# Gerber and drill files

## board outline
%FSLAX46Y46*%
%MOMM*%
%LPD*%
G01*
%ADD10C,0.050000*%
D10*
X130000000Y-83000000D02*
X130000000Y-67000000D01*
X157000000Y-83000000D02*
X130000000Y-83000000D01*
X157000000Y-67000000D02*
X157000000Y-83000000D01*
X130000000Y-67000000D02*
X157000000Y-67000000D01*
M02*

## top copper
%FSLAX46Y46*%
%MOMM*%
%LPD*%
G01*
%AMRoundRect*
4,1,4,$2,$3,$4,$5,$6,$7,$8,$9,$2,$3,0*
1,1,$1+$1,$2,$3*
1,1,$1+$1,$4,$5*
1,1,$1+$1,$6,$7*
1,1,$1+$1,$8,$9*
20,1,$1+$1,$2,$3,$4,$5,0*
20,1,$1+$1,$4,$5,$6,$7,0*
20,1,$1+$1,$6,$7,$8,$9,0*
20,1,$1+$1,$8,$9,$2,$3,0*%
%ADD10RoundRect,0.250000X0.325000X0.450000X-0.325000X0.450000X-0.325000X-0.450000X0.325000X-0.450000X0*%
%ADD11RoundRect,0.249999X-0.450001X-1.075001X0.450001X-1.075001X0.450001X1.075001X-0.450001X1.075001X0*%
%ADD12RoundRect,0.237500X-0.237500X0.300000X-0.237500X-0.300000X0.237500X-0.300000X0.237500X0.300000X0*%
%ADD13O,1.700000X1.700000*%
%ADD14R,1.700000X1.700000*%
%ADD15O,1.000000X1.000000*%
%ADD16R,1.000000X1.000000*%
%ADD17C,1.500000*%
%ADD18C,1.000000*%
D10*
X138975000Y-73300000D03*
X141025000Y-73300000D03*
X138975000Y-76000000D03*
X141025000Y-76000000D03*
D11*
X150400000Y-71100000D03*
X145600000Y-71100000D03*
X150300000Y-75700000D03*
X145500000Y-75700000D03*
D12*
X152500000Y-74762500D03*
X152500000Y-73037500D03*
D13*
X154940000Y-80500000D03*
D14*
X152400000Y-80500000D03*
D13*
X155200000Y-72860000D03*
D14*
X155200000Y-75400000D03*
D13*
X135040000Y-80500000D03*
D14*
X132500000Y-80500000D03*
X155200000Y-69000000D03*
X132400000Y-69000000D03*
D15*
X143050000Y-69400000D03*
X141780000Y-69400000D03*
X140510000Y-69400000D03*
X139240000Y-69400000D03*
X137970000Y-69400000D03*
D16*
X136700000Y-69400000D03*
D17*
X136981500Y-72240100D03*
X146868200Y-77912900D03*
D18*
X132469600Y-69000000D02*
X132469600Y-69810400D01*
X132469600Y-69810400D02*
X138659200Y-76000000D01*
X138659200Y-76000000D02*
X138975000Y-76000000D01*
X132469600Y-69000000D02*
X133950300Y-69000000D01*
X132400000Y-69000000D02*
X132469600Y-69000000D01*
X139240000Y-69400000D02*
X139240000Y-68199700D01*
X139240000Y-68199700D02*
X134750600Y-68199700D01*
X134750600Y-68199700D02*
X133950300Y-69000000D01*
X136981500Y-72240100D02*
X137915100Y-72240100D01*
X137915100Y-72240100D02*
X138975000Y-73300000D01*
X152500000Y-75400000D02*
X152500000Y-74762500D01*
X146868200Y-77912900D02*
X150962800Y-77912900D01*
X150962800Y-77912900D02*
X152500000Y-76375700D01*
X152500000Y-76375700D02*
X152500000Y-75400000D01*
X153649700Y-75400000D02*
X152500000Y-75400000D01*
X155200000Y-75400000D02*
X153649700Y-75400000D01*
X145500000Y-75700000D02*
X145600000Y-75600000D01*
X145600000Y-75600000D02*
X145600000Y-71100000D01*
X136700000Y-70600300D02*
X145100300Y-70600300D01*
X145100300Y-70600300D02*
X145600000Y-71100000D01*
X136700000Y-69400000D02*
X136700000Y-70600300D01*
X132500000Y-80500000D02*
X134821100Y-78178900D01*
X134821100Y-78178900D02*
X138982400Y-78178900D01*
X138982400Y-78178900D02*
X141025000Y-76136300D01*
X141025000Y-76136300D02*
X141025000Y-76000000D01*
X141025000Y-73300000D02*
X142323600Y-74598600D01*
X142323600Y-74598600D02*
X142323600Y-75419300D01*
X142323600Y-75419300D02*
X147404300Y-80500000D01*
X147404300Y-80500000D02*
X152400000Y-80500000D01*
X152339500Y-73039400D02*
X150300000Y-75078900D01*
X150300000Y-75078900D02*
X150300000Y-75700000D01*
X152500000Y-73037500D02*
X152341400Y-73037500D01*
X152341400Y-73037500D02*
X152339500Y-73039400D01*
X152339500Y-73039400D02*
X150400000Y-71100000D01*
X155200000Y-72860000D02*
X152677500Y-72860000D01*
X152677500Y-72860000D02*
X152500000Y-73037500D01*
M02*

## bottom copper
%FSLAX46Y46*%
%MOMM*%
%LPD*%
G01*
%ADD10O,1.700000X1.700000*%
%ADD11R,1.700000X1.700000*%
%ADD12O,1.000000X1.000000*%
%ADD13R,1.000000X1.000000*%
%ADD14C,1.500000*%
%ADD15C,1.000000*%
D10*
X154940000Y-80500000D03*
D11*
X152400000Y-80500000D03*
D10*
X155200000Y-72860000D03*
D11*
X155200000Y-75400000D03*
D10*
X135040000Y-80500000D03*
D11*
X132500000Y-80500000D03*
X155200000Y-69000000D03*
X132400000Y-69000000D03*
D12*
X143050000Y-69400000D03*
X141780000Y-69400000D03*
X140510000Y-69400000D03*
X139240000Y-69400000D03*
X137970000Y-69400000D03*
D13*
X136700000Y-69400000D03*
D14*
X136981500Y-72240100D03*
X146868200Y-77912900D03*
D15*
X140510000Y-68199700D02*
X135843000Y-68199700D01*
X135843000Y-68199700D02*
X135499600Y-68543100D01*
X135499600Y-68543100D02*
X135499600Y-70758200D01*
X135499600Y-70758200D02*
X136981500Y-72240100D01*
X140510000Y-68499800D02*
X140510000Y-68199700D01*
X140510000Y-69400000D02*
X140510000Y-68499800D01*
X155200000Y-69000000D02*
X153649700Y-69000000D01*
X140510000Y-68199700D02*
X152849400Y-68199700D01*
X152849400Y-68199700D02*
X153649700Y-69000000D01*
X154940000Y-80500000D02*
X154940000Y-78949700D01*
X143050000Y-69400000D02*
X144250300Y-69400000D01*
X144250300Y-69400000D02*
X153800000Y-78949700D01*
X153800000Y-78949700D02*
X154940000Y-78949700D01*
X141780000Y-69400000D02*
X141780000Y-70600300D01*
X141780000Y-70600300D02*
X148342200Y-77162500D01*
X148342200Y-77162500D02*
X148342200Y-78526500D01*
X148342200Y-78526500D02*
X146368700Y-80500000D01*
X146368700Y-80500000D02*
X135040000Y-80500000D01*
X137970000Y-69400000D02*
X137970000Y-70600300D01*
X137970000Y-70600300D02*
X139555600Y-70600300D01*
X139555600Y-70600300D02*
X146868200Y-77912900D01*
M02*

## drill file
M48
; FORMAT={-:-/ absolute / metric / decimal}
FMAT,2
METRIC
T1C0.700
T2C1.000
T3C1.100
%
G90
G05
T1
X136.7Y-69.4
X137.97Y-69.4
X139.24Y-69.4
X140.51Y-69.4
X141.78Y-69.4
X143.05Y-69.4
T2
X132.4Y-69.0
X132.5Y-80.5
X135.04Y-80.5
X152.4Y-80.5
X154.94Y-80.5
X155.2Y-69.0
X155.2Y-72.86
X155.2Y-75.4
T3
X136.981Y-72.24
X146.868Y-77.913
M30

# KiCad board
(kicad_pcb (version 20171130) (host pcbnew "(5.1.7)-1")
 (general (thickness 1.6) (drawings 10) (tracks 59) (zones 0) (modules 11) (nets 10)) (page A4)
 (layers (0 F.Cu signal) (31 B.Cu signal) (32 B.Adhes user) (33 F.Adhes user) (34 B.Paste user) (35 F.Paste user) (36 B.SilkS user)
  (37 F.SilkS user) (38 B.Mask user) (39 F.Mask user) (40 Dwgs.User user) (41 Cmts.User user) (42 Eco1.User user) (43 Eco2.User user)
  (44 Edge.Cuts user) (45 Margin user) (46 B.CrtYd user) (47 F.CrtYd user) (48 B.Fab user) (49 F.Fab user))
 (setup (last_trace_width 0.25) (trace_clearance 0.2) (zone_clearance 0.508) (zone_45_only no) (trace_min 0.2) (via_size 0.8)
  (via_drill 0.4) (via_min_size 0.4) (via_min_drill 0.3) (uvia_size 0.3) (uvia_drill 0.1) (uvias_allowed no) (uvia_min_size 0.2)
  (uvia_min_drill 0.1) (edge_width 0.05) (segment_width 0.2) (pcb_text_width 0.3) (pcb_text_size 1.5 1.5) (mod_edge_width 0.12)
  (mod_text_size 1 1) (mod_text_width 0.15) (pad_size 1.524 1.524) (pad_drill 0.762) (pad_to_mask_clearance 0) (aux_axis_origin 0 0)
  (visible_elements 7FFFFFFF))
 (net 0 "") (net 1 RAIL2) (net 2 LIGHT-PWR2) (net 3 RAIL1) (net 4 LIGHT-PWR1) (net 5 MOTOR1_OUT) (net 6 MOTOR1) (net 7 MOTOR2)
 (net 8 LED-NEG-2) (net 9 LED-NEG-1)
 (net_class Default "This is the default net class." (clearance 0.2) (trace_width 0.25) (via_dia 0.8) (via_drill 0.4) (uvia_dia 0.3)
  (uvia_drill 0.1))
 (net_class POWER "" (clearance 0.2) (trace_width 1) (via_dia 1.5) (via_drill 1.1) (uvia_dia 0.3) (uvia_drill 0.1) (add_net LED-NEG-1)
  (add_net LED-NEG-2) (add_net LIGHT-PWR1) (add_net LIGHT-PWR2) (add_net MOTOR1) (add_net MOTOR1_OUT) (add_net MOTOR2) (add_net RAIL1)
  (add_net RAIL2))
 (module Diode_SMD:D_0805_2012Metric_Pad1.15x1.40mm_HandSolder (layer F.Cu) (at 140 73.3 180)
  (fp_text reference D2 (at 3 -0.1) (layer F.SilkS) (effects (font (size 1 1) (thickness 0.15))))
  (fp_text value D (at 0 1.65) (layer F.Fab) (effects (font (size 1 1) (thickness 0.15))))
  (pad 2 smd roundrect (at 1.025 0 180) (size 1.15 1.4) (layers F.Cu F.Paste F.Mask) (roundrect_rratio 0.217391) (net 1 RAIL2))
  (pad 1 smd roundrect (at -1.025 0 180) (size 1.15 1.4) (layers F.Cu F.Paste F.Mask) (roundrect_rratio 0.217391) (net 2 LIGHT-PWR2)))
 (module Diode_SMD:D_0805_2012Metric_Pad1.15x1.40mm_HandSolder (layer F.Cu) (at 140 76 180)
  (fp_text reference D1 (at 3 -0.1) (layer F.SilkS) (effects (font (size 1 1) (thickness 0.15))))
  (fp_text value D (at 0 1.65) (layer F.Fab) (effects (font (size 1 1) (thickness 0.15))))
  (pad 2 smd roundrect (at 1.025 0 180) (size 1.15 1.4) (layers F.Cu F.Paste F.Mask) (roundrect_rratio 0.217391) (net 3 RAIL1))
  (pad 1 smd roundrect (at -1.025 0 180) (size 1.15 1.4) (layers F.Cu F.Paste F.Mask) (roundrect_rratio 0.217391) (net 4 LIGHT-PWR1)))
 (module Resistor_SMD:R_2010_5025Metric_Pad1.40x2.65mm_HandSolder (layer F.Cu) (at 148 71.1)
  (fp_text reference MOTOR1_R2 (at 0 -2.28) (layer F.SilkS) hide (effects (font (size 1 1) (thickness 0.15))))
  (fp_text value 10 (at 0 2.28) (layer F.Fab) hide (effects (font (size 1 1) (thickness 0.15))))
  (pad 2 smd roundrect (at 2.4 0) (size 1.4 2.65) (layers F.Cu F.Paste F.Mask) (roundrect_rratio 0.178571) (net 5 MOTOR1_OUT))
  (pad 1 smd roundrect (at -2.4 0) (size 1.4 2.65) (layers F.Cu F.Paste F.Mask) (roundrect_rratio 0.178571) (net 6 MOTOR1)))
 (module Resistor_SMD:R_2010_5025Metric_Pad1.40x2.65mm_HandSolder (layer F.Cu) (at 147.9 75.7)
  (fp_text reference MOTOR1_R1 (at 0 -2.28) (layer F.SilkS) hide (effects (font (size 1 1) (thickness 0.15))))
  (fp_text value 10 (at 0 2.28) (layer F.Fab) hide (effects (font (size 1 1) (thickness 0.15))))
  (pad 2 smd roundrect (at 2.4 0) (size 1.4 2.65) (layers F.Cu F.Paste F.Mask) (roundrect_rratio 0.178571) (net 5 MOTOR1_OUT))
  (pad 1 smd roundrect (at -2.4 0) (size 1.4 2.65) (layers F.Cu F.Paste F.Mask) (roundrect_rratio 0.178571) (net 6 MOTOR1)))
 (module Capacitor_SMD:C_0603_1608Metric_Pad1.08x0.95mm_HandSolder (layer F.Cu) (at 152.5 73.9 270)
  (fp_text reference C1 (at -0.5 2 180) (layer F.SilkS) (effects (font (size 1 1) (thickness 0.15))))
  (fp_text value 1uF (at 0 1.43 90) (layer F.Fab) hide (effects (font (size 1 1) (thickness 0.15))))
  (pad 2 smd roundrect (at 0.8625 0 270) (size 1.075 0.95) (layers F.Cu F.Paste F.Mask) (roundrect_rratio 0.25) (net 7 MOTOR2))
  (pad 1 smd roundrect (at -0.8625 0 270) (size 1.075 0.95) (layers F.Cu F.Paste F.Mask) (roundrect_rratio 0.25) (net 5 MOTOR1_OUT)))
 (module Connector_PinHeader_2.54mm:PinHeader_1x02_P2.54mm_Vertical (layer F.Cu) (at 152.4 80.5 90)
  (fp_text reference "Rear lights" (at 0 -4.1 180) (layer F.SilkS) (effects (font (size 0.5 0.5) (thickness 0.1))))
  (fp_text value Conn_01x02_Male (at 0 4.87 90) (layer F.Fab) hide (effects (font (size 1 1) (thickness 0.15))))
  (pad 2 thru_hole oval (at 0 2.54 90) (size 1.7 1.7) (drill 1) (layers *.Cu *.Mask) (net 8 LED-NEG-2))
  (pad 1 thru_hole rect (at 0 0 90) (size 1.7 1.7) (drill 1) (layers *.Cu *.Mask) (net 2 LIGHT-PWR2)))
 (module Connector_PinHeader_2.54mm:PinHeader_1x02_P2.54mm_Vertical (layer F.Cu) (at 155.2 75.4 180)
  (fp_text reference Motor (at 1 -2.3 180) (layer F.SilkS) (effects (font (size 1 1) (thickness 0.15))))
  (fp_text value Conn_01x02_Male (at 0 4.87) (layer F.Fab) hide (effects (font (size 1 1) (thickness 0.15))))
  (pad 2 thru_hole oval (at 0 2.54 180) (size 1.7 1.7) (drill 1) (layers *.Cu *.Mask) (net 5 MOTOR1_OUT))
  (pad 1 thru_hole rect (at 0 0 180) (size 1.7 1.7) (drill 1) (layers *.Cu *.Mask) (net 7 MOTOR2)))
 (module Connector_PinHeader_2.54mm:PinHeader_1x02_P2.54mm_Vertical (layer F.Cu) (at 132.5 80.5 90)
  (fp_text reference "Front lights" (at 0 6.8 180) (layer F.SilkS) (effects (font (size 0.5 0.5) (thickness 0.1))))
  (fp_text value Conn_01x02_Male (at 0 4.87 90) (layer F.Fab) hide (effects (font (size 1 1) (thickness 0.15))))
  (pad 2 thru_hole oval (at 0 2.54 90) (size 1.7 1.7) (drill 1) (layers *.Cu *.Mask) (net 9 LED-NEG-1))
  (pad 1 thru_hole rect (at 0 0 90) (size 1.7 1.7) (drill 1) (layers *.Cu *.Mask) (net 4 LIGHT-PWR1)))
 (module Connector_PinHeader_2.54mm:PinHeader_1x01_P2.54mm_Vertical (layer F.Cu) (at 155.2 69)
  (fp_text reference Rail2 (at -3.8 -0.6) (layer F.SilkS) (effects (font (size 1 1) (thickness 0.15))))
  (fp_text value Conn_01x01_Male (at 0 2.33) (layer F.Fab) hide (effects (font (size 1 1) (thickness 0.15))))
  (pad 1 thru_hole rect (at 0 0) (size 1.7 1.7) (drill 1) (layers *.Cu *.Mask) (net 1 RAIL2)))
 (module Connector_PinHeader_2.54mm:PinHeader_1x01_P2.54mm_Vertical (layer F.Cu) (at 132.4 69)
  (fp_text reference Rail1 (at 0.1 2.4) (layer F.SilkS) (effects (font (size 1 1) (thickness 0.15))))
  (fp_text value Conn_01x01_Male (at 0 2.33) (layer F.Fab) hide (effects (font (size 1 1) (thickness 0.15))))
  (pad 1 thru_hole rect (at 0 0) (size 1.7 1.7) (drill 1) (layers *.Cu *.Mask) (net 3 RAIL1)))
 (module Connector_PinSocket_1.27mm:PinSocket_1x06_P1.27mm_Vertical (layer F.Cu) (at 136.7 69.4 90)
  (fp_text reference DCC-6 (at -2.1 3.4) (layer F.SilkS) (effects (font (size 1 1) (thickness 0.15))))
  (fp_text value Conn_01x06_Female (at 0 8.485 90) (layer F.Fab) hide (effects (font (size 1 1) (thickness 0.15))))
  (pad 6 thru_hole oval (at 0 6.35 90) (size 1 1) (drill 0.7) (layers *.Cu *.Mask) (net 8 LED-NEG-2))
  (pad 5 thru_hole oval (at 0 5.08 90) (size 1 1) (drill 0.7) (layers *.Cu *.Mask) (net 9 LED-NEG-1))
  (pad 4 thru_hole oval (at 0 3.81 90) (size 1 1) (drill 0.7) (layers *.Cu *.Mask) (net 1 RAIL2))
  (pad 3 thru_hole oval (at 0 2.54 90) (size 1 1) (drill 0.7) (layers *.Cu *.Mask) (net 3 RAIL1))
  (pad 2 thru_hole oval (at 0 1.27 90) (size 1 1) (drill 0.7) (layers *.Cu *.Mask) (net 7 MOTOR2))
  (pad 1 thru_hole rect (at 0 0 90) (size 1 1) (drill 0.7) (layers *.Cu *.Mask) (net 6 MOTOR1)))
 (gr_line (start 130 83) (end 130 67) (layer Edge.Cuts) (width 0.05))
 (gr_line (start 157 83) (end 130 83) (layer Edge.Cuts) (width 0.05))
 (gr_line (start 157 67) (end 157 83) (layer Edge.Cuts) (width 0.05))
 (gr_line (start 130 67) (end 157 67) (layer Edge.Cuts) (width 0.05))
 (segment (start 132.4696 69) (end 132.4696 69.8104) (width 1) (layer F.Cu) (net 3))
 (segment (start 132.4696 69.8104) (end 138.6592 76) (width 1) (layer F.Cu) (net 3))
 (segment (start 138.6592 76) (end 138.975 76) (width 1) (layer F.Cu) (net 3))
 (segment (start 132.4696 69) (end 133.9503 69) (width 1) (layer F.Cu) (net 3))
 (segment (start 132.4 69) (end 132.4696 69) (width 1) (layer F.Cu) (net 3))
 (segment (start 139.24 69.4) (end 139.24 68.1997) (width 1) (layer F.Cu) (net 3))
 (segment (start 139.24 68.1997) (end 134.7506 68.1997) (width 1) (layer F.Cu) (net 3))
 (segment (start 134.7506 68.1997) (end 133.9503 69) (width 1) (layer F.Cu) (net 3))
 (segment (start 136.9815 72.2401) (end 137.9151 72.2401) (width 1) (layer F.Cu) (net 1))
 (segment (start 137.9151 72.2401) (end 138.975 73.3) (width 1) (layer F.Cu) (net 1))
 (segment (start 140.51 68.1997) (end 135.843 68.1997) (width 1) (layer B.Cu) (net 1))
 (segment (start 135.843 68.1997) (end 135.4996 68.5431) (width 1) (layer B.Cu) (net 1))
 (segment (start 135.4996 68.5431) (end 135.4996 70.7582) (width 1) (layer B.Cu) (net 1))
 (segment (start 135.4996 70.7582) (end 136.9815 72.2401) (width 1) (layer B.Cu) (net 1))
 (segment (start 140.51 68.4998) (end 140.51 68.1997) (width 1) (layer B.Cu) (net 1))
 (segment (start 140.51 69.4) (end 140.51 68.4998) (width 1) (layer B.Cu) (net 1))
 (segment (start 155.2 69) (end 153.6497 69) (width 1) (layer B.Cu) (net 1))
 (segment (start 140.51 68.1997) (end 152.8494 68.1997) (width 1) (layer B.Cu) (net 1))
 (segment (start 152.8494 68.1997) (end 153.6497 69) (width 1) (layer B.Cu) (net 1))
 (via (at 136.9815 72.2401) (size 1.5) (drill 1.1) (layers F.Cu B.Cu) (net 1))
 (segment (start 154.94 80.5) (end 154.94 78.9497) (width 1) (layer B.Cu) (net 8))
 (segment (start 143.05 69.4) (end 144.2503 69.4) (width 1) (layer B.Cu) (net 8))
 (segment (start 144.2503 69.4) (end 153.8 78.9497) (width 1) (layer B.Cu) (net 8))
 (segment (start 153.8 78.9497) (end 154.94 78.9497) (width 1) (layer B.Cu) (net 8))
 (segment (start 141.78 69.4) (end 141.78 70.6003) (width 1) (layer B.Cu) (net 9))
 (segment (start 141.78 70.6003) (end 148.3422 77.1625) (width 1) (layer B.Cu) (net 9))
 (segment (start 148.3422 77.1625) (end 148.3422 78.5265) (width 1) (layer B.Cu) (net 9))
 (segment (start 148.3422 78.5265) (end 146.3687 80.5) (width 1) (layer B.Cu) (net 9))
 (segment (start 146.3687 80.5) (end 135.04 80.5) (width 1) (layer B.Cu) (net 9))
 (segment (start 152.5 75.4) (end 152.5 74.7625) (width 1) (layer F.Cu) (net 7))
 (segment (start 146.8682 77.9129) (end 150.9628 77.9129) (width 1) (layer F.Cu) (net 7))
 (segment (start 150.9628 77.9129) (end 152.5 76.3757) (width 1) (layer F.Cu) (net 7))
 (segment (start 152.5 76.3757) (end 152.5 75.4) (width 1) (layer F.Cu) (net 7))
 (segment (start 153.6497 75.4) (end 152.5 75.4) (width 1) (layer F.Cu) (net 7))
 (segment (start 155.2 75.4) (end 153.6497 75.4) (width 1) (layer F.Cu) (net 7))
 (segment (start 137.97 69.4) (end 137.97 70.6003) (width 1) (layer B.Cu) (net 7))
 (segment (start 137.97 70.6003) (end 139.5556 70.6003) (width 1) (layer B.Cu) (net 7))
 (segment (start 139.5556 70.6003) (end 146.8682 77.9129) (width 1) (layer B.Cu) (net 7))
 (via (at 146.8682 77.9129) (size 1.5) (drill 1.1) (layers F.Cu B.Cu) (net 7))
 (segment (start 145.5 75.7) (end 145.6 75.6) (width 1) (layer F.Cu) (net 6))
 (segment (start 145.6 75.6) (end 145.6 71.1) (width 1) (layer F.Cu) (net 6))
 (segment (start 136.7 70.6003) (end 145.1003 70.6003) (width 1) (layer F.Cu) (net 6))
 (segment (start 145.1003 70.6003) (end 145.6 71.1) (width 1) (layer F.Cu) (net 6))
 (segment (start 136.7 69.4) (end 136.7 70.6003) (width 1) (layer F.Cu) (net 6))
 (segment (start 132.5 80.5) (end 134.8211 78.1789) (width 1) (layer F.Cu) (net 4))
 (segment (start 134.8211 78.1789) (end 138.9824 78.1789) (width 1) (layer F.Cu) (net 4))
 (segment (start 138.9824 78.1789) (end 141.025 76.1363) (width 1) (layer F.Cu) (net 4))
 (segment (start 141.025 76.1363) (end 141.025 76) (width 1) (layer F.Cu) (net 4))
 (segment (start 141.025 73.3) (end 142.3236 74.5986) (width 1) (layer F.Cu) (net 2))
 (segment (start 142.3236 74.5986) (end 142.3236 75.4193) (width 1) (layer F.Cu) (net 2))
 (segment (start 142.3236 75.4193) (end 147.4043 80.5) (width 1) (layer F.Cu) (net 2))
 (segment (start 147.4043 80.5) (end 152.4 80.5) (width 1) (layer F.Cu) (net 2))
 (segment (start 152.3395 73.0394) (end 150.3 75.0789) (width 1) (layer F.Cu) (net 5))
 (segment (start 150.3 75.0789) (end 150.3 75.7) (width 1) (layer F.Cu) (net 5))
 (segment (start 152.5 73.0375) (end 152.3414 73.0375) (width 1) (layer F.Cu) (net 5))
 (segment (start 152.3414 73.0375) (end 152.3395 73.0394) (width 1) (layer F.Cu) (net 5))
 (segment (start 152.3395 73.0394) (end 150.4 71.1) (width 1) (layer F.Cu) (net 5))
 (segment (start 155.2 72.86) (end 152.6775 72.86) (width 1) (layer F.Cu) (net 5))
 (segment (start 152.6775 72.86) (end 152.5 73.0375) (width 1) (layer F.Cu) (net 5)))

